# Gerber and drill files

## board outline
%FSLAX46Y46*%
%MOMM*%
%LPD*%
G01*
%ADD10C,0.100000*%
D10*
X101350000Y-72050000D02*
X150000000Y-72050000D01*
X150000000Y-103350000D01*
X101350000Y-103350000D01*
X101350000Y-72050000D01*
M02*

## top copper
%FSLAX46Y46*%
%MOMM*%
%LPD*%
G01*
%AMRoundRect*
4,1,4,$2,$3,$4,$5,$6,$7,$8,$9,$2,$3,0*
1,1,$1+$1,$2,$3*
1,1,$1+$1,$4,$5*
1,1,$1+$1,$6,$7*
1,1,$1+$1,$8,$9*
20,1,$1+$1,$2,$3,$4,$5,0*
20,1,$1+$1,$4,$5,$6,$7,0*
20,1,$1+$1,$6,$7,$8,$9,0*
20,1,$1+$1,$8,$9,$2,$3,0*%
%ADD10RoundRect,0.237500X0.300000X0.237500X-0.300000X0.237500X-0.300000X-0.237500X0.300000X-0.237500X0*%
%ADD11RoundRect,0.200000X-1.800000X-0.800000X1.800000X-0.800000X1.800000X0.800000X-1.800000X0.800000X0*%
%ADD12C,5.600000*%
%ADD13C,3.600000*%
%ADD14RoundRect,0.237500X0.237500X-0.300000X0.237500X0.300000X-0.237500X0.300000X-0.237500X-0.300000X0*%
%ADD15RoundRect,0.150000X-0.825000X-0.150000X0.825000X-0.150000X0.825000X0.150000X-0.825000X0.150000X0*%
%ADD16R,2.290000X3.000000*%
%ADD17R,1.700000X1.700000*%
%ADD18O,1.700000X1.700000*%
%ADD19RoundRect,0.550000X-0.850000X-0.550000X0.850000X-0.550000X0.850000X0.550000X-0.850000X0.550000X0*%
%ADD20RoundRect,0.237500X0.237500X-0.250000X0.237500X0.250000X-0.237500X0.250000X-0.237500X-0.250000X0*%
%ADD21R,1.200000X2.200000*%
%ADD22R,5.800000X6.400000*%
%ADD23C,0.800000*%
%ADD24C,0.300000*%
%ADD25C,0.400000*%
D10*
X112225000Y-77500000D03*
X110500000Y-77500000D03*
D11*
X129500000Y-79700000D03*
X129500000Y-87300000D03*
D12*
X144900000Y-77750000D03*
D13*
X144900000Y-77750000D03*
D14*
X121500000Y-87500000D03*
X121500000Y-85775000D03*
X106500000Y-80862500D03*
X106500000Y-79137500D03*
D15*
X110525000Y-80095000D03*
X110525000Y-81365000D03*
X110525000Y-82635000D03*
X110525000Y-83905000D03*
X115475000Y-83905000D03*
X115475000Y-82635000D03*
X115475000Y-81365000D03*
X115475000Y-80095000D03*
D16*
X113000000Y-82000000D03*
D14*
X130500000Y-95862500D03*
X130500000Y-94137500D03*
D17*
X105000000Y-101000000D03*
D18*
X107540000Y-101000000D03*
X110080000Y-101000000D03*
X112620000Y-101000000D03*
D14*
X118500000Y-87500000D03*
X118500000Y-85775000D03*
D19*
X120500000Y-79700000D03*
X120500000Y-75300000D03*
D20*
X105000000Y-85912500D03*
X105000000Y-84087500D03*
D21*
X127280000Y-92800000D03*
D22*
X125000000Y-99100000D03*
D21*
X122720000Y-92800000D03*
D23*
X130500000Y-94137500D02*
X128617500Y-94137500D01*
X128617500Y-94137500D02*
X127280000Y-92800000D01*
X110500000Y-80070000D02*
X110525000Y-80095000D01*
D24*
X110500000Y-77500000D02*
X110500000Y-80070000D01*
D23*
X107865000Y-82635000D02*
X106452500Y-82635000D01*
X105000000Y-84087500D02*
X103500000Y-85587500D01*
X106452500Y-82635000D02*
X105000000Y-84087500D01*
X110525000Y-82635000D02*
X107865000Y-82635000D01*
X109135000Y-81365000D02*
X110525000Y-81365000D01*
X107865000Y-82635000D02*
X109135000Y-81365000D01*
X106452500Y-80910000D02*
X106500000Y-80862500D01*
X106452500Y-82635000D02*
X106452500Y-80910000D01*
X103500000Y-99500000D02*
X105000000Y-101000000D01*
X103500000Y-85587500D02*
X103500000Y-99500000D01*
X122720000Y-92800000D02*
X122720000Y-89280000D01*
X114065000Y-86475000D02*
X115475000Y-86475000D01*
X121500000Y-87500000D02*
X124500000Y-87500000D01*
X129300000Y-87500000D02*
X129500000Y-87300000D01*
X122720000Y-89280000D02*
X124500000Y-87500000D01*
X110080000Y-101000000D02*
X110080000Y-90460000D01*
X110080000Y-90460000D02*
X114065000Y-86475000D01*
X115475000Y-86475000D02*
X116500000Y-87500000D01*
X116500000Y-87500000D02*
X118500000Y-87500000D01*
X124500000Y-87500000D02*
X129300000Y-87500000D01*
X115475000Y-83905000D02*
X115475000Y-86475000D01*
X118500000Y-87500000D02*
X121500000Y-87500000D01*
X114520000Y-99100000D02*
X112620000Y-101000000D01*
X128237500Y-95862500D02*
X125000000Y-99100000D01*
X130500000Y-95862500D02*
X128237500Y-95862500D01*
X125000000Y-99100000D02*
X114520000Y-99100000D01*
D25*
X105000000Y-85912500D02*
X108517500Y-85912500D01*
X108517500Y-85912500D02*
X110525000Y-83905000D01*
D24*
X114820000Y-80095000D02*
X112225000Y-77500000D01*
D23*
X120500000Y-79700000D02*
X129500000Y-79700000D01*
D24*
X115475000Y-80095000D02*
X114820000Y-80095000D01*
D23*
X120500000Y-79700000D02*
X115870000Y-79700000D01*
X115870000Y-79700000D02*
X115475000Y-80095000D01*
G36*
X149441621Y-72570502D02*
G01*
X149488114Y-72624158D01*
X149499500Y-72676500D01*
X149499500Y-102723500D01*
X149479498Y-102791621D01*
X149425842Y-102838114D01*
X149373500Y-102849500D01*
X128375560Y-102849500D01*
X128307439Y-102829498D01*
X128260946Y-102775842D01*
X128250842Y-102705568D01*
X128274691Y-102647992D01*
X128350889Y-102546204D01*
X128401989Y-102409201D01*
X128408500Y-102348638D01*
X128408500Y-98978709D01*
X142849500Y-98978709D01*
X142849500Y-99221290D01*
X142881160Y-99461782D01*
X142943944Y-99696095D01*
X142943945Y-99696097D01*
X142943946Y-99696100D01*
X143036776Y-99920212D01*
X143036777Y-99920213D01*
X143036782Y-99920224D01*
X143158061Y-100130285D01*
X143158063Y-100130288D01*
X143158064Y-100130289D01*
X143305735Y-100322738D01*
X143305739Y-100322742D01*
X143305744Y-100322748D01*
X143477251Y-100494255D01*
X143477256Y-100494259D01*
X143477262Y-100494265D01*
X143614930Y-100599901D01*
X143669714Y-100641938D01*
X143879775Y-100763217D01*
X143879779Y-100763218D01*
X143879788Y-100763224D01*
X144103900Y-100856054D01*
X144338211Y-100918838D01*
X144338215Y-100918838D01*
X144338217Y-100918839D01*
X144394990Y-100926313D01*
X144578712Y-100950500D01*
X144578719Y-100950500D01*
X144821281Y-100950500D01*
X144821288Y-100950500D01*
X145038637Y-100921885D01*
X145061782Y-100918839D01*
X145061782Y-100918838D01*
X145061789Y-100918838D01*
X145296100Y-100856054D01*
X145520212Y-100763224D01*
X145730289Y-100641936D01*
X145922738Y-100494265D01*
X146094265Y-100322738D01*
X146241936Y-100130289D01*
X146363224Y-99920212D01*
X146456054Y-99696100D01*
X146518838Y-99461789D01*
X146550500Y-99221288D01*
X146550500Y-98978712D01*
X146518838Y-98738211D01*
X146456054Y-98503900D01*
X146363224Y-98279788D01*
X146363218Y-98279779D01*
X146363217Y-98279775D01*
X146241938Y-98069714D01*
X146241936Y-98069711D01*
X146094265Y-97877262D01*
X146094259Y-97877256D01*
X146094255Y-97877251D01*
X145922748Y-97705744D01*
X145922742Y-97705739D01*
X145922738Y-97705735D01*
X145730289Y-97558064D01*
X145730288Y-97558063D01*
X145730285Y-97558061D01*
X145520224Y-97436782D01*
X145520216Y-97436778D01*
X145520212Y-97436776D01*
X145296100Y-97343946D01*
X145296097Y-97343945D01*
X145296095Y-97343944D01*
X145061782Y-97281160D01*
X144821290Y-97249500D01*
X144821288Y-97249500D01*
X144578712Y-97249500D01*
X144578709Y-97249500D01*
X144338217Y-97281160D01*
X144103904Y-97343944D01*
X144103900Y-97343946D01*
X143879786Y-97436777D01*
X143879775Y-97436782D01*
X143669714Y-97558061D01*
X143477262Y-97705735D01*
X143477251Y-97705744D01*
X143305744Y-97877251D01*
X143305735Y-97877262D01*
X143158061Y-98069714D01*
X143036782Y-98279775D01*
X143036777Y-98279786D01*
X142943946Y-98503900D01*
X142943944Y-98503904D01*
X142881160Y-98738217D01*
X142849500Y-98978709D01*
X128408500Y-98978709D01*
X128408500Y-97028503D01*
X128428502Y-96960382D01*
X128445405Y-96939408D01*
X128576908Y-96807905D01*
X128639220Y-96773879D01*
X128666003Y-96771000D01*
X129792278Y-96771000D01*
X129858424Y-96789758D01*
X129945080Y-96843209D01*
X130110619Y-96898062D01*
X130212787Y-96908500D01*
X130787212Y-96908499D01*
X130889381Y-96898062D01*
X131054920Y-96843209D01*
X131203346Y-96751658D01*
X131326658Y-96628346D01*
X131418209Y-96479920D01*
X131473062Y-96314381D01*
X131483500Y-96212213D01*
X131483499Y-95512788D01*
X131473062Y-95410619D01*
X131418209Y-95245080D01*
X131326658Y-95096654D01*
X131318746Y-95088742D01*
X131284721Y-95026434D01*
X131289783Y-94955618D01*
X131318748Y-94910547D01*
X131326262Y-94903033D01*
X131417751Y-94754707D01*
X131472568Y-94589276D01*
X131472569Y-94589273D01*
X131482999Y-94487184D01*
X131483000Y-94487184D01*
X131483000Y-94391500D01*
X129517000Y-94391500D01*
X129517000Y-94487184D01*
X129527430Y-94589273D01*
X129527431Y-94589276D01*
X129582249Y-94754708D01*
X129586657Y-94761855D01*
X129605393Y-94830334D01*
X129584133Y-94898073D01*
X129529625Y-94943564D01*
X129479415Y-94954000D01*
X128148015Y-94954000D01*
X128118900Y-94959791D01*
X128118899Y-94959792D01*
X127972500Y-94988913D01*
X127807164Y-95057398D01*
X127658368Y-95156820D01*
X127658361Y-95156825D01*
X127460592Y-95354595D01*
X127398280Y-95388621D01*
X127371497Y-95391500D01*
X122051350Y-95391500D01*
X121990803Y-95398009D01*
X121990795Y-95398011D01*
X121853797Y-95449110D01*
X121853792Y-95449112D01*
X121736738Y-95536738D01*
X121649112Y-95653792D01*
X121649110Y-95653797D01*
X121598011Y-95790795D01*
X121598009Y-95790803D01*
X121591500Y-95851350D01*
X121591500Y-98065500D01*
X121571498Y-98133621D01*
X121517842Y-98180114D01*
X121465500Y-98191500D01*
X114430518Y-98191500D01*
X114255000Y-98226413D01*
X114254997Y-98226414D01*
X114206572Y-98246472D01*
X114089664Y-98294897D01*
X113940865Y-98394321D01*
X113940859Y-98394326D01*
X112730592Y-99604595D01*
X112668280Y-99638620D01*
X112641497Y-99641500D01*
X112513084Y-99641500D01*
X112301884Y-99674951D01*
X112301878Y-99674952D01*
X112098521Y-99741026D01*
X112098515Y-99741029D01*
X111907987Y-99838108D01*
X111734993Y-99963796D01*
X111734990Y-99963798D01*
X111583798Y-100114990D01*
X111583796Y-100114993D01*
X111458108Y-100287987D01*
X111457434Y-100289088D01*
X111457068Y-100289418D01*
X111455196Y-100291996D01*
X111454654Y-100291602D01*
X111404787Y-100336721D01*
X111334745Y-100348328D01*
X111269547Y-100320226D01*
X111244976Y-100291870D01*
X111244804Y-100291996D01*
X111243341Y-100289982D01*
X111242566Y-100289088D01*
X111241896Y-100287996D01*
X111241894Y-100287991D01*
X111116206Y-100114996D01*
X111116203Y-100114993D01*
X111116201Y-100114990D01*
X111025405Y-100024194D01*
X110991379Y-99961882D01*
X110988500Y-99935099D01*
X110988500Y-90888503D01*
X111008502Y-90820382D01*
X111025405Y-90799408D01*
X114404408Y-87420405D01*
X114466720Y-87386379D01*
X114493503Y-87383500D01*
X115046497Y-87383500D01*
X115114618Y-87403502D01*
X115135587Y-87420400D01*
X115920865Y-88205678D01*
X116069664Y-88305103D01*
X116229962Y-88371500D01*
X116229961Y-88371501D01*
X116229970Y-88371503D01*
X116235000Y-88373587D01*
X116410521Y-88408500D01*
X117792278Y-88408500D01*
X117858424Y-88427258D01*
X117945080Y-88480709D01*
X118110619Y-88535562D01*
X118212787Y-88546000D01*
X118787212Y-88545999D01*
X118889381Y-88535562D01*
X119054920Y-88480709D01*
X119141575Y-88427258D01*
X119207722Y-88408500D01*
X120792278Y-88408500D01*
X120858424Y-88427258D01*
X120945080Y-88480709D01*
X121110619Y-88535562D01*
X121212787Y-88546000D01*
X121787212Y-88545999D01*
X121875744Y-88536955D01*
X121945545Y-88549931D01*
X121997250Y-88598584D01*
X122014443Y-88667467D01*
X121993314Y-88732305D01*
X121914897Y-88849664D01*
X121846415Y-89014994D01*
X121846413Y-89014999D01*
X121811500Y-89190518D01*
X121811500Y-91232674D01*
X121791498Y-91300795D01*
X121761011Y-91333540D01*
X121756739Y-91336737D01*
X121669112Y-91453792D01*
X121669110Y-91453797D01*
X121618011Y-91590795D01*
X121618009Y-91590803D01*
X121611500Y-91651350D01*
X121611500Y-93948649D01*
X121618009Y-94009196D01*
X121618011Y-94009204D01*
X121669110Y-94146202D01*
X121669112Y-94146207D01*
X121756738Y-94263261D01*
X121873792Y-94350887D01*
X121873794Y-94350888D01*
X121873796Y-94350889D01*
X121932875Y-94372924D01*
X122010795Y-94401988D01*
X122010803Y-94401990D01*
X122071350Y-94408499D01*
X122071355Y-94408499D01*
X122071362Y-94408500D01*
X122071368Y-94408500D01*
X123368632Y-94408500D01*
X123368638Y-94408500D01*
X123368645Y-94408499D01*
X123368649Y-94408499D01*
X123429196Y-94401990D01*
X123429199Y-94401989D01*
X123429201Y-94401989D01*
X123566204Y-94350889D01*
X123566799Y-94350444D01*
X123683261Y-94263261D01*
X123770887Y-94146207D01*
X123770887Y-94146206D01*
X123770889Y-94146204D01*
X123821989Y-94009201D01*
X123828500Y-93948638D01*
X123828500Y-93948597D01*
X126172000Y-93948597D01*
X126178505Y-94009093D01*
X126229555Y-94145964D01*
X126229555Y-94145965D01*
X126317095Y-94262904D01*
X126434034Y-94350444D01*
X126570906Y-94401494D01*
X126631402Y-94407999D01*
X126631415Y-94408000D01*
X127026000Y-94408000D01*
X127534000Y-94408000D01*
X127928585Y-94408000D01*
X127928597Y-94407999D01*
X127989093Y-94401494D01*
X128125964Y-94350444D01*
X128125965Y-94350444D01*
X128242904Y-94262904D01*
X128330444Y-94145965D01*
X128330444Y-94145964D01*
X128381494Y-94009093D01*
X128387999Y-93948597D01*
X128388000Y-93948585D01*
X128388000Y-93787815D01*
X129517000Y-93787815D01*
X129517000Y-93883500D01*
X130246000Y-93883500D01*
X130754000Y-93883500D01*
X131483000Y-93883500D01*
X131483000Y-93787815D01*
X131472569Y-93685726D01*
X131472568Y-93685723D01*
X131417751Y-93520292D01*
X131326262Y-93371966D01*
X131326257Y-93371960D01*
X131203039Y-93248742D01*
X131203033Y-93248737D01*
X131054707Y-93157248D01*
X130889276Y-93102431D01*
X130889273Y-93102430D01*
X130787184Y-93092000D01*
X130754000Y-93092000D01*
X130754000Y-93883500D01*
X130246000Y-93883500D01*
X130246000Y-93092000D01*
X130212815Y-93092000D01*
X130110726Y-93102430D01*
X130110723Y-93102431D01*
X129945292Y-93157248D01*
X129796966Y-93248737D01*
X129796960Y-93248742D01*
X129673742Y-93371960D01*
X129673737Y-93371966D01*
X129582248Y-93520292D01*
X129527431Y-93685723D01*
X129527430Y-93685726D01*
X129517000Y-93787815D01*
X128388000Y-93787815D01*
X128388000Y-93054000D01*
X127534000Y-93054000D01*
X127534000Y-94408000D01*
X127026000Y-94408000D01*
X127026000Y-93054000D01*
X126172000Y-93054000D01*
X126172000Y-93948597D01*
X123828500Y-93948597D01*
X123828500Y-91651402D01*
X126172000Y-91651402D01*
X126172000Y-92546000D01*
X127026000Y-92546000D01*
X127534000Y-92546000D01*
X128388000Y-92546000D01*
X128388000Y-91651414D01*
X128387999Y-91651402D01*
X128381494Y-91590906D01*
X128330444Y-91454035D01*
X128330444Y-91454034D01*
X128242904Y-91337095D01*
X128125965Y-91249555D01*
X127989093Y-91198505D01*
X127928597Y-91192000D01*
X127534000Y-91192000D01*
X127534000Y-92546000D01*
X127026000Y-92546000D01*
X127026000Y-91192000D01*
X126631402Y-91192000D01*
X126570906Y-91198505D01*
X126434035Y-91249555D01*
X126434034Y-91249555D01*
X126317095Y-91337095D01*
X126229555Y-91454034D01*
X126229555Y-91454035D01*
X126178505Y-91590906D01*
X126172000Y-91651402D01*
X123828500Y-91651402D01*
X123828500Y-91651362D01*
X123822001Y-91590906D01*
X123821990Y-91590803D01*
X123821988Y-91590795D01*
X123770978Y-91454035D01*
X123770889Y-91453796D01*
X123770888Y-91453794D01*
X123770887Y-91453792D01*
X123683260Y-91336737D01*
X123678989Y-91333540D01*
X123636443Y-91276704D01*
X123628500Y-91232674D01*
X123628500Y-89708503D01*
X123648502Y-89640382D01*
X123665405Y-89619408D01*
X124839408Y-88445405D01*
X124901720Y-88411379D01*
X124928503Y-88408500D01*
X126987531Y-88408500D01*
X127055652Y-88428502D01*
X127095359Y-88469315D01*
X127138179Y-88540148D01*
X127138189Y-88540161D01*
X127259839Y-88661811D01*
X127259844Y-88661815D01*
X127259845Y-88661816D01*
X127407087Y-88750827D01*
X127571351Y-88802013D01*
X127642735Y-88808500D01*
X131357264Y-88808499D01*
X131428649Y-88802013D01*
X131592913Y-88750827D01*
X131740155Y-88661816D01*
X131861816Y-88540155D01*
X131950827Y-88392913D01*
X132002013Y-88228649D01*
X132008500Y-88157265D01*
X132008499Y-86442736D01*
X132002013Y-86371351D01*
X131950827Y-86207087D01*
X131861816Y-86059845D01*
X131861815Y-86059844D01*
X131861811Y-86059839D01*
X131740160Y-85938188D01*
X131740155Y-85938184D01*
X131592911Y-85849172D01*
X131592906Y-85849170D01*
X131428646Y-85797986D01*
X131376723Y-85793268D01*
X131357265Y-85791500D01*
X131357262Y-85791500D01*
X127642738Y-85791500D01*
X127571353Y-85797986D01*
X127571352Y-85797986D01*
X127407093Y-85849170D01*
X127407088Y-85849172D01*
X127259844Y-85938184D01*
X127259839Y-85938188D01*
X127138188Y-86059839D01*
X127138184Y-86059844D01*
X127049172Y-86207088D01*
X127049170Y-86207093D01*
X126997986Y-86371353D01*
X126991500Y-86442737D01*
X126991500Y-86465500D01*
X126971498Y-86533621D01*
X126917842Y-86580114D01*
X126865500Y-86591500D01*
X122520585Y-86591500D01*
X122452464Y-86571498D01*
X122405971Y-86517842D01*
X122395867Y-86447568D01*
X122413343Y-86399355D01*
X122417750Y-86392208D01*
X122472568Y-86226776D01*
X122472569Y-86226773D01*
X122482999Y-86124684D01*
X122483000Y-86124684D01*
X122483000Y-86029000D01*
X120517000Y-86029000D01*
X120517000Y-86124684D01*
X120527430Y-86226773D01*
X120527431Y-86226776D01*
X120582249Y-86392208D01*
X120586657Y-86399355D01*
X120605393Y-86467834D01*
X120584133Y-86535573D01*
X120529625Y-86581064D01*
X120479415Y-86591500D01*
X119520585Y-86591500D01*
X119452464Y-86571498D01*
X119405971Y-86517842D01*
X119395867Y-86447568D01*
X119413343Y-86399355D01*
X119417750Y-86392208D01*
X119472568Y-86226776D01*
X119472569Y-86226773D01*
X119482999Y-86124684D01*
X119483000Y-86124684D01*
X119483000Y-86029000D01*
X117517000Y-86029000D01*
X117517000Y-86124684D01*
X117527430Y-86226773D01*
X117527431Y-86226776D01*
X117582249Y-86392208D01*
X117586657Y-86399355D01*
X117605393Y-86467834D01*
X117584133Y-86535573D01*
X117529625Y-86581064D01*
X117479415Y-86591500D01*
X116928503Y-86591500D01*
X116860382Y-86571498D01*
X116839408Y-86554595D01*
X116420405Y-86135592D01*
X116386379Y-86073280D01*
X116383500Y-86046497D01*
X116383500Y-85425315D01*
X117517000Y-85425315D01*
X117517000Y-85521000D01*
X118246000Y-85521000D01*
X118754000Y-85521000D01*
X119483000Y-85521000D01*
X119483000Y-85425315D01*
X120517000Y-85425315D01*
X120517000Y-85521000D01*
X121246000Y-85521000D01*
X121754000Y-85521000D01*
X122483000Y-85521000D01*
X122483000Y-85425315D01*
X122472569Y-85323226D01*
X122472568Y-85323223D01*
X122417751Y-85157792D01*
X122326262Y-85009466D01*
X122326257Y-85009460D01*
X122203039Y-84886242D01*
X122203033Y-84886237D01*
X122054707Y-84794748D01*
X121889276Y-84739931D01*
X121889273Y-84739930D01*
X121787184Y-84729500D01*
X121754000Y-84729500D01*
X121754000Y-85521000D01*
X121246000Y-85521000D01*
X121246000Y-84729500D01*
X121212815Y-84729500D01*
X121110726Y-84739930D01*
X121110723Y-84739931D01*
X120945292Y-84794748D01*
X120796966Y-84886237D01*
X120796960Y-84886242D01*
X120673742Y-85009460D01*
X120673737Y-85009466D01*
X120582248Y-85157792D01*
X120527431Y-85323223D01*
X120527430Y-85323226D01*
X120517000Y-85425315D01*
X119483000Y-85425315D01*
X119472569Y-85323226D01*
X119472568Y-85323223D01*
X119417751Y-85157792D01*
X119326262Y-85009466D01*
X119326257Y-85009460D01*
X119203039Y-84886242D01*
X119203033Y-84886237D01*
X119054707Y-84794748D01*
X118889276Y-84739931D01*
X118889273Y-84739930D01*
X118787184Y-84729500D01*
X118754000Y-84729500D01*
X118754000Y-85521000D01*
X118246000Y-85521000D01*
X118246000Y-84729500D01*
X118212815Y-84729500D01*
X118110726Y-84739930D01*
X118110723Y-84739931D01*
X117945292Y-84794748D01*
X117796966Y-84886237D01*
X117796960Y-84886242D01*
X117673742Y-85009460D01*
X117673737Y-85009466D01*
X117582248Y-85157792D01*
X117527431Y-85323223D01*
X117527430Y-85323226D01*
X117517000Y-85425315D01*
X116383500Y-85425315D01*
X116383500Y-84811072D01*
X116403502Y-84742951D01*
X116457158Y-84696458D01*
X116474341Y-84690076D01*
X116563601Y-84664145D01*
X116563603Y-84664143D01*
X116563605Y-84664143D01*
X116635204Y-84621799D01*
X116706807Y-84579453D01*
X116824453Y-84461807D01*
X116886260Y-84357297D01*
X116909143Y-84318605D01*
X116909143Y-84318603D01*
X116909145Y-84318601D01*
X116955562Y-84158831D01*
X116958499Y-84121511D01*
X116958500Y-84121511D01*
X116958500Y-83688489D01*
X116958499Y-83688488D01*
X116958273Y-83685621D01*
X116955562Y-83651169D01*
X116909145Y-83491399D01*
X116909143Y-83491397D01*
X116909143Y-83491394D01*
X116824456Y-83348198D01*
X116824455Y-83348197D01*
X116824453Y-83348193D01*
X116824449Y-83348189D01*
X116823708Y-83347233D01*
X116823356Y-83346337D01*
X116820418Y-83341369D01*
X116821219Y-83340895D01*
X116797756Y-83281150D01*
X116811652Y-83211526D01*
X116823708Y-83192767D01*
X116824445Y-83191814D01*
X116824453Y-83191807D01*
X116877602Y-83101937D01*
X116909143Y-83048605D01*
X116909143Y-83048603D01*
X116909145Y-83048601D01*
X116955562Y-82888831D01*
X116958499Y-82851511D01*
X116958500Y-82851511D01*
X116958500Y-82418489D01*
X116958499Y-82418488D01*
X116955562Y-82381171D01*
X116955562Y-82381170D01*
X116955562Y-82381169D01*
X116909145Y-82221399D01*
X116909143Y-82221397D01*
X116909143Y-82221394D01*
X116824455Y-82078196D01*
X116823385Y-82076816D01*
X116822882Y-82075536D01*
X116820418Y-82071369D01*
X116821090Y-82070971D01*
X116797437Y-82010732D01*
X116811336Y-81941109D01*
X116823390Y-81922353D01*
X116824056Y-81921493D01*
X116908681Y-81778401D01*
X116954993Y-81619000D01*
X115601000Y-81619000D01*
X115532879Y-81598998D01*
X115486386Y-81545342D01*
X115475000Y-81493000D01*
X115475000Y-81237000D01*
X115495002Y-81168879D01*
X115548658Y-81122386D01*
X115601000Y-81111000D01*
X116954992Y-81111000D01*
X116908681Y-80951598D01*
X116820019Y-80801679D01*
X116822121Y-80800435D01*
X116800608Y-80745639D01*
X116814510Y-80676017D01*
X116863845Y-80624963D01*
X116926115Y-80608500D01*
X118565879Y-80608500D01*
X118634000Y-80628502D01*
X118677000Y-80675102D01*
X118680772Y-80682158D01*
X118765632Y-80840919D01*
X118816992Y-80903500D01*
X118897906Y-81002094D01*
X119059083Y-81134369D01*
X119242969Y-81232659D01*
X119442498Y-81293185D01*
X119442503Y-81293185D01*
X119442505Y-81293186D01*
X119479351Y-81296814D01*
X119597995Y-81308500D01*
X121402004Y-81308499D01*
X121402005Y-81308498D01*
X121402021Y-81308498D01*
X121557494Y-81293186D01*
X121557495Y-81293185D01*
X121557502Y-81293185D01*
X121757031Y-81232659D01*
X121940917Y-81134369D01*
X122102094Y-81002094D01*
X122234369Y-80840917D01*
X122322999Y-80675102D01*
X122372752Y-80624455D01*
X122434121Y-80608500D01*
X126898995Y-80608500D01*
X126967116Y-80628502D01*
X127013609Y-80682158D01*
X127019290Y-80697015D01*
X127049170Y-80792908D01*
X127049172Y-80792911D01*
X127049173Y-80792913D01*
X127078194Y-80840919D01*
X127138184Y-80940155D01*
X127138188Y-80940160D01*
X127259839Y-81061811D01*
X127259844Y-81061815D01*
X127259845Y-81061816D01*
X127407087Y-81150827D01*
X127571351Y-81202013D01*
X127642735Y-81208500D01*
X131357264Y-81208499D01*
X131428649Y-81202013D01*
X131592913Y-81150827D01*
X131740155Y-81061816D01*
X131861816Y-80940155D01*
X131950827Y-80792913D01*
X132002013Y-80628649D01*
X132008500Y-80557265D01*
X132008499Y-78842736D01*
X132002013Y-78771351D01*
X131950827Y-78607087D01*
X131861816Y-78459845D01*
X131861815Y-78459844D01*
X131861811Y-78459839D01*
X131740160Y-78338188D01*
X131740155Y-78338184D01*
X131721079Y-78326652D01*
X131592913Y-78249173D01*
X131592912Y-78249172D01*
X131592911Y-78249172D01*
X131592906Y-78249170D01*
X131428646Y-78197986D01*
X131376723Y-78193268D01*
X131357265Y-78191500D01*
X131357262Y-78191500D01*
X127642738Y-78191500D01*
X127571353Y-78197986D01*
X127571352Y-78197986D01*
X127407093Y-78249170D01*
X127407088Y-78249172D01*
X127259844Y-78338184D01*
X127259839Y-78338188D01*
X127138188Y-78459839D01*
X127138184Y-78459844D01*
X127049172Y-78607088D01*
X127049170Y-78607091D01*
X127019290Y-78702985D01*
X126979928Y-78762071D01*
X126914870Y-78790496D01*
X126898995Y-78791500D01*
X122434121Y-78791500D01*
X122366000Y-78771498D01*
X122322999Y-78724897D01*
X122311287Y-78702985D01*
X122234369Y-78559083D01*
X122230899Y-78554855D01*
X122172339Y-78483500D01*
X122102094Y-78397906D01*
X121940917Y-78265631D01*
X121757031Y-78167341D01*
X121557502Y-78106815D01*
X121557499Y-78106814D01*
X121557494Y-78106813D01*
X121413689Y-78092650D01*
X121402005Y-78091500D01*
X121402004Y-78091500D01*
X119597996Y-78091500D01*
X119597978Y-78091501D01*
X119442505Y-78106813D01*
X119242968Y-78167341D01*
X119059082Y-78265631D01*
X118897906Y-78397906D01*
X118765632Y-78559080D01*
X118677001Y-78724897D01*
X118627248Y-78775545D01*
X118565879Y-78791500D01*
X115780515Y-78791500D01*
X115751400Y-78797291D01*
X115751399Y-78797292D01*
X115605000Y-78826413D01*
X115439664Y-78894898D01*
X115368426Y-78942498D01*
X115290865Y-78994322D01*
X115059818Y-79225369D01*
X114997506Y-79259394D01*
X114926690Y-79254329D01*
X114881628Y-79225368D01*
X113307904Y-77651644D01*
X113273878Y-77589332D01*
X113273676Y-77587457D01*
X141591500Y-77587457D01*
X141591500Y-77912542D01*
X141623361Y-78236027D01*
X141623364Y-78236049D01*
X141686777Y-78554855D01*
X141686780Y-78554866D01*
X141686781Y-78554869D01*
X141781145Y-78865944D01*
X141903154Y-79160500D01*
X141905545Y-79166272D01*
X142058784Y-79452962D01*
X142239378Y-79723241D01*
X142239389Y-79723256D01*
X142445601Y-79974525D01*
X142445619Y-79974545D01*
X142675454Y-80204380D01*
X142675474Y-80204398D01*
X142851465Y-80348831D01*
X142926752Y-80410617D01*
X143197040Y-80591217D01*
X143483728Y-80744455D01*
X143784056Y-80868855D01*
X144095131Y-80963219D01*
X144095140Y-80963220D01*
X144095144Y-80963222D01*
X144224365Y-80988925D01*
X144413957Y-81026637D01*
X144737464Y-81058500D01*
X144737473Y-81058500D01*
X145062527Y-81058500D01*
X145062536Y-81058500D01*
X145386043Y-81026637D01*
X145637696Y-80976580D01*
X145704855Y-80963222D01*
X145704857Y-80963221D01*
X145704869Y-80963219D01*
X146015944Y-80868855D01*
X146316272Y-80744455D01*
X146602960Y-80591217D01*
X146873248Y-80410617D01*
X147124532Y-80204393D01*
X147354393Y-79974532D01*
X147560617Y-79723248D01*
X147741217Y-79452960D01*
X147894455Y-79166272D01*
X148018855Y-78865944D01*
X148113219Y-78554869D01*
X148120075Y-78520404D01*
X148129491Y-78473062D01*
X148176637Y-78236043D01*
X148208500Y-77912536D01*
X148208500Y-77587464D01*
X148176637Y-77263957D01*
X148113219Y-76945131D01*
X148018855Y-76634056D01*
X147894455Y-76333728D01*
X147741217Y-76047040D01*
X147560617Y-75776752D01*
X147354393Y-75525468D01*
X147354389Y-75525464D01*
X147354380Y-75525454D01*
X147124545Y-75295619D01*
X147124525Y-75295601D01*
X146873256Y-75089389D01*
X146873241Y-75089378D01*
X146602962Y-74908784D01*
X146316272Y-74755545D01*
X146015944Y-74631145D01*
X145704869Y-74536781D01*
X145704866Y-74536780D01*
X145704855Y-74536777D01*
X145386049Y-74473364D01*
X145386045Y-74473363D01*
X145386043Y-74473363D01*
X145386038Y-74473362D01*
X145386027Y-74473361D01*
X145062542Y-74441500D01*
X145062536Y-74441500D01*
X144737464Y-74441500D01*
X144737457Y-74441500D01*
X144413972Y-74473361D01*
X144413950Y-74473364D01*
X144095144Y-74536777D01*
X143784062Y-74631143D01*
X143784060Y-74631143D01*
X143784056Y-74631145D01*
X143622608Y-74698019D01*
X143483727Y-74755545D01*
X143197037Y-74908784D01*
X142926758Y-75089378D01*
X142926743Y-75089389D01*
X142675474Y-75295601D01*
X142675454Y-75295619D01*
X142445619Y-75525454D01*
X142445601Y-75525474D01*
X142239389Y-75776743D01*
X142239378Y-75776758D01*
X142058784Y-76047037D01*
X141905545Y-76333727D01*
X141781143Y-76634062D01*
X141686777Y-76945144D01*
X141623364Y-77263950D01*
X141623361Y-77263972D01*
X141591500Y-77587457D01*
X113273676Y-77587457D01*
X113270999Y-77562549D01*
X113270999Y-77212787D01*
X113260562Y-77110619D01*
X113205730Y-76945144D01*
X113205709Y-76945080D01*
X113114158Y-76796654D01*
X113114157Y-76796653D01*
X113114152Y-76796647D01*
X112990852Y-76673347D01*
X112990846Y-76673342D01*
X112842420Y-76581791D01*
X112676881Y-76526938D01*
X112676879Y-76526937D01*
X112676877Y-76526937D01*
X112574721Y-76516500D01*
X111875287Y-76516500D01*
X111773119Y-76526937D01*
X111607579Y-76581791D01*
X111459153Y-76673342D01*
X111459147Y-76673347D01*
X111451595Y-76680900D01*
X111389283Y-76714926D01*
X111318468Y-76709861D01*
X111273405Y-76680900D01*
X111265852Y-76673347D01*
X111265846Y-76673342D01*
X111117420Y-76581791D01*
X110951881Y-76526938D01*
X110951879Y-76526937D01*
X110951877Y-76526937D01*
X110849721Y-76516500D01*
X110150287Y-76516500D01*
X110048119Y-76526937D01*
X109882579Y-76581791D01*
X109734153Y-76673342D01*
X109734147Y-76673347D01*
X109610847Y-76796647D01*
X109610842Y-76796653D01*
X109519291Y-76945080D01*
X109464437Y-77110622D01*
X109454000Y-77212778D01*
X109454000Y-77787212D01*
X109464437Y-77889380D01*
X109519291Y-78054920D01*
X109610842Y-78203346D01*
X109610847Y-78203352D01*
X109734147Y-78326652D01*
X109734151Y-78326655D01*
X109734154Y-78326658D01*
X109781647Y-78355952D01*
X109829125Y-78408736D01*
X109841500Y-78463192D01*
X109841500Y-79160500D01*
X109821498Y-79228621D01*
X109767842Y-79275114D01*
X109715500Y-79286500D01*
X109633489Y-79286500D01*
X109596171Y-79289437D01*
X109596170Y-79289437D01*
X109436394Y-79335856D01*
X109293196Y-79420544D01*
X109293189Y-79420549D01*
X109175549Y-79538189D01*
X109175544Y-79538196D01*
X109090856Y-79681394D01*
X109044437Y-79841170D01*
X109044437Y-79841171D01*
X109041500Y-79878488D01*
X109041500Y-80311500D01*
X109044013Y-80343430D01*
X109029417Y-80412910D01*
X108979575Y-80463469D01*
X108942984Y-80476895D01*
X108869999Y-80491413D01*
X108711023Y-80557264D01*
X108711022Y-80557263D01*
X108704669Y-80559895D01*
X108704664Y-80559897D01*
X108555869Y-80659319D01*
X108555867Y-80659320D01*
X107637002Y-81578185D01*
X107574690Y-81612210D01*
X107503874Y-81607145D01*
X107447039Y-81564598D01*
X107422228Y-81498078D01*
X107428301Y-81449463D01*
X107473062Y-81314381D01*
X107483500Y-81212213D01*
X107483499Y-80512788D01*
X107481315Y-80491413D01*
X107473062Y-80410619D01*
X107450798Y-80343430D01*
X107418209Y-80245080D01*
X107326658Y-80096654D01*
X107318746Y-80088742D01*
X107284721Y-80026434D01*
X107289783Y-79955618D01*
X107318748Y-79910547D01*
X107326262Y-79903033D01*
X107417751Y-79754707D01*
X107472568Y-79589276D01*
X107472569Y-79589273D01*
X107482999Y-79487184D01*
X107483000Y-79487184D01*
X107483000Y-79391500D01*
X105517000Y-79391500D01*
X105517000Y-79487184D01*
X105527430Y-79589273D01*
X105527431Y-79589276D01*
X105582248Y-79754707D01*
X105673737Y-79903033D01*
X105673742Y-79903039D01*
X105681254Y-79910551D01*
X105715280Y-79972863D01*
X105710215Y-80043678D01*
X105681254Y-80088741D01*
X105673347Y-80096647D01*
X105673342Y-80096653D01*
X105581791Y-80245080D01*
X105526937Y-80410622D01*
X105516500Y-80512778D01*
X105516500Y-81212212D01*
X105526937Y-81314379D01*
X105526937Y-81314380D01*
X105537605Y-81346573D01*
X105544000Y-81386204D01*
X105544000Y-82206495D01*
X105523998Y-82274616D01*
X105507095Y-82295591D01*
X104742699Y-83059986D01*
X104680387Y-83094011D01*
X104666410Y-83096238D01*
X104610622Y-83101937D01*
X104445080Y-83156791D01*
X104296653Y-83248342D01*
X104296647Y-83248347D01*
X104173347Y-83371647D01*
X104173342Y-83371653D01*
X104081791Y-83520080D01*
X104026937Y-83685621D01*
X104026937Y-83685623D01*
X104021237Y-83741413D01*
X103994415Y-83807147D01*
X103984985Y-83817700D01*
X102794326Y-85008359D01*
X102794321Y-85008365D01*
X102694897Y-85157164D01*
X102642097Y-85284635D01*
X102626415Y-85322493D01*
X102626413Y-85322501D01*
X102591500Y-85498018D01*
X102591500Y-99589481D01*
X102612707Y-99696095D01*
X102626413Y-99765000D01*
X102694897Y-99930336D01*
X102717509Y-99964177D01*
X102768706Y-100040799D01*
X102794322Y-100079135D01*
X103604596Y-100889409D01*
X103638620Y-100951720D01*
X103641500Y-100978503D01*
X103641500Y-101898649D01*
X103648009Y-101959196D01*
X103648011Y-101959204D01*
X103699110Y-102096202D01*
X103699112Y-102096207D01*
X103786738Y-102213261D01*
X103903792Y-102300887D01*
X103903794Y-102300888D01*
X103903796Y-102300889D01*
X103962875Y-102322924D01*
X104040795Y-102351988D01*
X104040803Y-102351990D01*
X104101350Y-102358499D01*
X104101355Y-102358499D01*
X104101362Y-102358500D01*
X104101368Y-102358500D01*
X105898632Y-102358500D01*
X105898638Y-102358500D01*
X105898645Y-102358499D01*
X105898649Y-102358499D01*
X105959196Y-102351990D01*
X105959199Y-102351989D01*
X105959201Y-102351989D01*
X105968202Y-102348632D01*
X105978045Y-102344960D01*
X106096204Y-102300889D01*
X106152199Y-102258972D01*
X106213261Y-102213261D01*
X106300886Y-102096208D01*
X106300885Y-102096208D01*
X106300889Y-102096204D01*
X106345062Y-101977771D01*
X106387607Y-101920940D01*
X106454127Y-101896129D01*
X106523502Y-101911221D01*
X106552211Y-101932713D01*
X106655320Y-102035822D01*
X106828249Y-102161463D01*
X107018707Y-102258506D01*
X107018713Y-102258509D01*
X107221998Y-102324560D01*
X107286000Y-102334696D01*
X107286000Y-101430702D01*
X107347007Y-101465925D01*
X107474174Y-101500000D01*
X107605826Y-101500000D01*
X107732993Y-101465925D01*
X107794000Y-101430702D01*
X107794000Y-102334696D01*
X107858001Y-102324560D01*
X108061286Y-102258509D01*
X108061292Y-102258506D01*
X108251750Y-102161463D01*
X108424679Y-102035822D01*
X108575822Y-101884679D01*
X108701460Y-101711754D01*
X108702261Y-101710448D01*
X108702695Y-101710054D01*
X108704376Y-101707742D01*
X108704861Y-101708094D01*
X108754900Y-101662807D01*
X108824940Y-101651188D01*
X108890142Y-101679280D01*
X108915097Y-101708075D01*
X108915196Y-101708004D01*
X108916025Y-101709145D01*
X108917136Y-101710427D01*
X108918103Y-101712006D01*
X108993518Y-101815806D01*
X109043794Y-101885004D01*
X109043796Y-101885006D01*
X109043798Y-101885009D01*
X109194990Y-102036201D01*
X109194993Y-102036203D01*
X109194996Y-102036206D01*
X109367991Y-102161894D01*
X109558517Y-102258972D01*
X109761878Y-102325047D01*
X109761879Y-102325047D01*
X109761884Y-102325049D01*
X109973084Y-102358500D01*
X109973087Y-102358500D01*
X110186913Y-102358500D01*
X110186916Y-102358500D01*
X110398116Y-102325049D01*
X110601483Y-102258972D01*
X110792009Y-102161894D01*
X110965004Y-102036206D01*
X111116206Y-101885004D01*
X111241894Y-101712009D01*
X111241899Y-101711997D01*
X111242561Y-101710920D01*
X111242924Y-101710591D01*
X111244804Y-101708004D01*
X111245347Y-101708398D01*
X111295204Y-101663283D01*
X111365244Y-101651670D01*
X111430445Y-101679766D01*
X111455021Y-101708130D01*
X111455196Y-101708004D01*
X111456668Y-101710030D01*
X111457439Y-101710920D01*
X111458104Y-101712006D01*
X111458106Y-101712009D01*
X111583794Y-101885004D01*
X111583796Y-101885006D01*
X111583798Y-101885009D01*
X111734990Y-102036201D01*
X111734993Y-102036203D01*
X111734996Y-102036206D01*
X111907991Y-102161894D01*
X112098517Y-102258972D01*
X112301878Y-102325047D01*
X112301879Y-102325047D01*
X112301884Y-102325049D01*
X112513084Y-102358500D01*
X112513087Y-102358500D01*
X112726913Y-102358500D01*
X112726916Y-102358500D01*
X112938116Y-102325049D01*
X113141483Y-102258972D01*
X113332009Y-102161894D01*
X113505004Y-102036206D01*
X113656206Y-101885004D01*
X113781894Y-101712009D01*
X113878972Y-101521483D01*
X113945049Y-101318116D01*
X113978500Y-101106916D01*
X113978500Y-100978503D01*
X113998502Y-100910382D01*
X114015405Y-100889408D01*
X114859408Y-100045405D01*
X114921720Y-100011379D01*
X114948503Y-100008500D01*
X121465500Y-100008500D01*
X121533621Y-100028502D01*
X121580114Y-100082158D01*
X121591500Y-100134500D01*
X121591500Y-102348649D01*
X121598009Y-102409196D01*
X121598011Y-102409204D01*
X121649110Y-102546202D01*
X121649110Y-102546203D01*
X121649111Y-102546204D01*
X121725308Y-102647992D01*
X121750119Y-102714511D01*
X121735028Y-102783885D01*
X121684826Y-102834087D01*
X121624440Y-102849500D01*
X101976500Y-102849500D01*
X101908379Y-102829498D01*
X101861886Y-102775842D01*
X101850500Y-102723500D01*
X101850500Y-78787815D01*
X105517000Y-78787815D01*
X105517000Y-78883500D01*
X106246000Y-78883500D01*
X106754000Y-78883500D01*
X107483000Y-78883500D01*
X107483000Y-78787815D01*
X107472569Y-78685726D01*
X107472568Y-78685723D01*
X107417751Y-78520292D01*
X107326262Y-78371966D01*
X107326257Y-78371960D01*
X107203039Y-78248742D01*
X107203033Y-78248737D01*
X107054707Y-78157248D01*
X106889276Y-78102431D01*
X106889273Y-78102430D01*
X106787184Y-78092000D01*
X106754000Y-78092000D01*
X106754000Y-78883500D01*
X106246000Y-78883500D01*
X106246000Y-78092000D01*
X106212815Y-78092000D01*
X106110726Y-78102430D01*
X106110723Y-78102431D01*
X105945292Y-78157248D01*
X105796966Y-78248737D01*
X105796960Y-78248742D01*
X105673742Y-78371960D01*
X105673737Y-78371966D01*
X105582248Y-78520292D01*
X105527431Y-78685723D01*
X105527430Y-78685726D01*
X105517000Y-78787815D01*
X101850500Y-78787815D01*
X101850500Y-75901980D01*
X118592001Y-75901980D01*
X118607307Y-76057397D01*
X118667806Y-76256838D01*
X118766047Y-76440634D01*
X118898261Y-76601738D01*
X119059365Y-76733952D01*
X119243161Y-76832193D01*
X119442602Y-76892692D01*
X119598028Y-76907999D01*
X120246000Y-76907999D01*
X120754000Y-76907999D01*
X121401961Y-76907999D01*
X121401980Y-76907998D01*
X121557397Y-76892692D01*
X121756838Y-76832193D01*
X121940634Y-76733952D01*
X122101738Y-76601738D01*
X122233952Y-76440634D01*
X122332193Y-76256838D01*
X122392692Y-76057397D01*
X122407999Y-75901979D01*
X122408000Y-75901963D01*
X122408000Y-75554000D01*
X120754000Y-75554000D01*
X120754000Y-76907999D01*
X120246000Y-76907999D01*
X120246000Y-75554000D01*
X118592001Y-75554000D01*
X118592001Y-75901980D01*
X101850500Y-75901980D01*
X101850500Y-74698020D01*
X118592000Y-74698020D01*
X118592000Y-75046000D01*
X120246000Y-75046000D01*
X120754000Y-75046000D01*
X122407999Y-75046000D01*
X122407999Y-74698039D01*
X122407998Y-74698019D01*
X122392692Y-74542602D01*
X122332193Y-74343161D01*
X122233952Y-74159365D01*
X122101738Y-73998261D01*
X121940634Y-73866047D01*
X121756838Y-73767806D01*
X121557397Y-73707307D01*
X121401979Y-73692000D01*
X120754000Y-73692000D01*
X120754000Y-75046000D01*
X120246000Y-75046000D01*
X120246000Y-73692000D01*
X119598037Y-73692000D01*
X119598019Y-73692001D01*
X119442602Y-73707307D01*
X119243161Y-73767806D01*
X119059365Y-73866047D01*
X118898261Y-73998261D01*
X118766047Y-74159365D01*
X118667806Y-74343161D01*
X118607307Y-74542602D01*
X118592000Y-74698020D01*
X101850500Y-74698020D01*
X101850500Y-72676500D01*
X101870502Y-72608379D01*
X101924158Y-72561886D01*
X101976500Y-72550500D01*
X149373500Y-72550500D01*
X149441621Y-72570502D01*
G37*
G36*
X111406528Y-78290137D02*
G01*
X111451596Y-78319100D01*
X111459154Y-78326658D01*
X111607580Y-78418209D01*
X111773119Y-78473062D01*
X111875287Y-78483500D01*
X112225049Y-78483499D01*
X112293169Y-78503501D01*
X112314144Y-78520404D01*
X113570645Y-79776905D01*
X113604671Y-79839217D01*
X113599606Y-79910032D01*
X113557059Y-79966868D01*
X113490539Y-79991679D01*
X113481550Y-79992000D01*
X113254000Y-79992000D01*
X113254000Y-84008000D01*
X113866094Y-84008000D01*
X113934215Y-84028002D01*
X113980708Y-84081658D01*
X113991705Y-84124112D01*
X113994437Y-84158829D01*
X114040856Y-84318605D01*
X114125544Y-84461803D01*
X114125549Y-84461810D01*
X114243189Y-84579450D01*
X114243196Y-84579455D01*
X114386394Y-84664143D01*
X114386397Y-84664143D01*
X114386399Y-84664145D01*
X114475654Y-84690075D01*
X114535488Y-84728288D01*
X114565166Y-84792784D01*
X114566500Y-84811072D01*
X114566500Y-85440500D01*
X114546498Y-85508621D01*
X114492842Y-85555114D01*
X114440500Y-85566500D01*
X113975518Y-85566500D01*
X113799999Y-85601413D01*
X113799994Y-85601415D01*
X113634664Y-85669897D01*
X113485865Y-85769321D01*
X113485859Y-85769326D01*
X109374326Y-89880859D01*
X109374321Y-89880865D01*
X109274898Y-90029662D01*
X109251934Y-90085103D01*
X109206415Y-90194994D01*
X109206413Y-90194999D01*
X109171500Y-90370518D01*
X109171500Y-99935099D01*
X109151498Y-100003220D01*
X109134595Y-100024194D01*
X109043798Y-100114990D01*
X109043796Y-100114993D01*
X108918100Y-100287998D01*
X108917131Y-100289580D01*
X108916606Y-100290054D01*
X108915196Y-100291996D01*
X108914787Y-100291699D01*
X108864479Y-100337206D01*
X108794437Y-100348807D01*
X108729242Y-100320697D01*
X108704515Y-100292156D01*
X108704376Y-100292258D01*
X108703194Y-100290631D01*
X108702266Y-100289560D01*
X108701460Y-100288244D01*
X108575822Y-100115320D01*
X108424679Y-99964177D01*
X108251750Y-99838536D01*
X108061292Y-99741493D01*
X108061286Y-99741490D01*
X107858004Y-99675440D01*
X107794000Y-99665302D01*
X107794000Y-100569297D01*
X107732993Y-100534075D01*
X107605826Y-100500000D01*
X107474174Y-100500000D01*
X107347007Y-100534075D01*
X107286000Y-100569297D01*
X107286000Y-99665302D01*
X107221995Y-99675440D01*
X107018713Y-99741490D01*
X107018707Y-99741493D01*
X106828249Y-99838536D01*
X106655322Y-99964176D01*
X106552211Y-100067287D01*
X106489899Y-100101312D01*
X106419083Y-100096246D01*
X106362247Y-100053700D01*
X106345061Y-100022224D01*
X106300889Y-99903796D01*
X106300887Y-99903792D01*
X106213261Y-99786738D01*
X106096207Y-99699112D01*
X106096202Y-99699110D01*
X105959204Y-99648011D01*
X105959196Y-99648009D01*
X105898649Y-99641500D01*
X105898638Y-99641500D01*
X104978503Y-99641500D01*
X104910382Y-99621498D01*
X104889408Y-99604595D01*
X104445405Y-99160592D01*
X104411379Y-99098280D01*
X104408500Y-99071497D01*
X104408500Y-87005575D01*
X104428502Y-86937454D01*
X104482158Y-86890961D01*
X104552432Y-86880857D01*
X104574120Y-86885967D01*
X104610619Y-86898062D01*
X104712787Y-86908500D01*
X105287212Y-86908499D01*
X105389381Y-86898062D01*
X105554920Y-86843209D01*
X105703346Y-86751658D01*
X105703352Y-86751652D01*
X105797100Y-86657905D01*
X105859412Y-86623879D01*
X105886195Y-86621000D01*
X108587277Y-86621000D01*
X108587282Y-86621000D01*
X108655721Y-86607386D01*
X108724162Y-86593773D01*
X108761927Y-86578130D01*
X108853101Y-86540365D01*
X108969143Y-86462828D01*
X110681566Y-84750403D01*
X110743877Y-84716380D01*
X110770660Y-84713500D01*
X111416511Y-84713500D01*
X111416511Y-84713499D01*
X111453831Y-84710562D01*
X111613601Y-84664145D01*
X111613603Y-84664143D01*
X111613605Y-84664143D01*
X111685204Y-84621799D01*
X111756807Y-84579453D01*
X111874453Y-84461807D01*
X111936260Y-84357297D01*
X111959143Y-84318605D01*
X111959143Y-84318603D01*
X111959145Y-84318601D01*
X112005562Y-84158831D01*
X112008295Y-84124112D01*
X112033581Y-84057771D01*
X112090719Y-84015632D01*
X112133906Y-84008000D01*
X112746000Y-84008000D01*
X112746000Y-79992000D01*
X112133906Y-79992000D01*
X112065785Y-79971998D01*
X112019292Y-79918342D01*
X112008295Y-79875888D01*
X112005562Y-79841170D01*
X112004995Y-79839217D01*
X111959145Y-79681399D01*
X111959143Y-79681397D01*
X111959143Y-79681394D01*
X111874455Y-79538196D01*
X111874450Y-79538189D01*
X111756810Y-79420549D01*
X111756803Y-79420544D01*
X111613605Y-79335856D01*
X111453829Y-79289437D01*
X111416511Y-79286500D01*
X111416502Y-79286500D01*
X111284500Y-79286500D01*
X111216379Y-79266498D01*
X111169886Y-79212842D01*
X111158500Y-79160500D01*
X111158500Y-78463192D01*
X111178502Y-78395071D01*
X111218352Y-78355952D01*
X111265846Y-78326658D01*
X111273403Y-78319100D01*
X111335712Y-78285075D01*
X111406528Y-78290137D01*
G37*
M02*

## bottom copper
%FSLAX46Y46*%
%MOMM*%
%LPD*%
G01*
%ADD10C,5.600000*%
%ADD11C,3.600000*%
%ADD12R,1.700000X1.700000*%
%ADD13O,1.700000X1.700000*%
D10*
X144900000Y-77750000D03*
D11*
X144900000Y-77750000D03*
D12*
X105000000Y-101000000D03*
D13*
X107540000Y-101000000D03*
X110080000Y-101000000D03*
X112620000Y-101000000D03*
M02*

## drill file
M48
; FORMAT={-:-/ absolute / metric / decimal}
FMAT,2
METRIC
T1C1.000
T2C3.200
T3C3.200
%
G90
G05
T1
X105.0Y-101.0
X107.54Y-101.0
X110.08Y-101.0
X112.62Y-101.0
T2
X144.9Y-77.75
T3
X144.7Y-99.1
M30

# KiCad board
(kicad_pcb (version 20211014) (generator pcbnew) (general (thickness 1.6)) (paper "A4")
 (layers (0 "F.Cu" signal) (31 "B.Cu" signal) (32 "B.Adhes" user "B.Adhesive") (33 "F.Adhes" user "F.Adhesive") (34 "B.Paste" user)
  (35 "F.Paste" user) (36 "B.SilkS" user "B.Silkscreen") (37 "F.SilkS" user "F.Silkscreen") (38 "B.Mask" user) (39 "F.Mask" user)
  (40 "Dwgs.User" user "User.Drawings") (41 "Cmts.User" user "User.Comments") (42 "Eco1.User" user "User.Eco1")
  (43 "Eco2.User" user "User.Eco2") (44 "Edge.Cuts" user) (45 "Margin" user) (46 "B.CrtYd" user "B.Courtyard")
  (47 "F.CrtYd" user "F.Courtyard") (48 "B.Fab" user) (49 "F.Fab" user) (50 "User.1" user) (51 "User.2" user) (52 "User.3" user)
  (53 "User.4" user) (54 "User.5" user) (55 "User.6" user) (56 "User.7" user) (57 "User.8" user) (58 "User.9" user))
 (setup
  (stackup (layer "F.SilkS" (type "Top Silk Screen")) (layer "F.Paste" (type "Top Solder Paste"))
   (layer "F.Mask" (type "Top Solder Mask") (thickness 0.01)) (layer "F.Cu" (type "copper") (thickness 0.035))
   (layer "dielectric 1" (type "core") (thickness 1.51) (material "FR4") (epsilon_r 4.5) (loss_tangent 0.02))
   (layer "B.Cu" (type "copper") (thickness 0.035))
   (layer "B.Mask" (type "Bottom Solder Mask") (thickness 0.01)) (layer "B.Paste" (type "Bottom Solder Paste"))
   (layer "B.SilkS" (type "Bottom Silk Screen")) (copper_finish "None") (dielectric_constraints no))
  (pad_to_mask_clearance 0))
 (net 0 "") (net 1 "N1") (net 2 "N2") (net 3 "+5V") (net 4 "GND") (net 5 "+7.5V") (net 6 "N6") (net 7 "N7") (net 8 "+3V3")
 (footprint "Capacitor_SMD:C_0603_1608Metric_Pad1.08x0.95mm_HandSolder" (layer "F.Cu") (at 111.3625 77.5 180)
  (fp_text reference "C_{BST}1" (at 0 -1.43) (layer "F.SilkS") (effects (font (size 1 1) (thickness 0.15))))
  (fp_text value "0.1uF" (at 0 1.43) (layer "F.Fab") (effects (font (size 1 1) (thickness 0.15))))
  (pad "1" smd roundrect (at -0.8625 0 180) (size 1.075 0.95) (layers "F.Cu" "F.Paste" "F.Mask") (roundrect_rratio 0.25) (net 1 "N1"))
  (pad "2" smd roundrect (at 0.8625 0 180) (size 1.075 0.95) (layers "F.Cu" "F.Paste" "F.Mask") (roundrect_rratio 0.25) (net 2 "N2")))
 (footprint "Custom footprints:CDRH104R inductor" (layer "F.Cu") (at 129.5 83.5)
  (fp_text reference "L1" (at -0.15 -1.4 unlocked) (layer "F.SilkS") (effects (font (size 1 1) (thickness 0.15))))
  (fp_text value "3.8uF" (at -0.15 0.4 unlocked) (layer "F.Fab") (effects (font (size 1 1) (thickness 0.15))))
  (pad "1" smd roundrect (at 0 -3.8) (size 4 2) (layers "F.Cu" "F.Paste" "F.Mask") (roundrect_rratio 0.1) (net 1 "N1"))
  (pad "2" smd roundrect (at 0 3.8) (size 4 2) (layers "F.Cu" "F.Paste" "F.Mask") (roundrect_rratio 0.1) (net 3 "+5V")))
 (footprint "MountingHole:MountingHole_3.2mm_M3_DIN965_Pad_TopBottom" (layer "F.Cu") (at 144.9 77.75)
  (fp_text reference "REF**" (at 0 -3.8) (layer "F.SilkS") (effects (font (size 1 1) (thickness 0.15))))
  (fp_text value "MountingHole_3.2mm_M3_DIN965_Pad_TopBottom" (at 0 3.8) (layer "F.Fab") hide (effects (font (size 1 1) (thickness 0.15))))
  (pad "1" connect circle (at 0 0) (size 5.6 5.6) (layers "B.Cu" "B.Mask"))
  (pad "1" connect circle (at 0 0) (size 5.6 5.6) (layers "F.Cu" "F.Mask"))
  (pad "1" thru_hole circle (at 0 0) (size 3.6 3.6) (drill 3.2) (layers *.Cu *.Mask)))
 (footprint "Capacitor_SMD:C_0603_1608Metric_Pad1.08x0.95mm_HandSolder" (layer "F.Cu") (at 121.5 86.6375 90)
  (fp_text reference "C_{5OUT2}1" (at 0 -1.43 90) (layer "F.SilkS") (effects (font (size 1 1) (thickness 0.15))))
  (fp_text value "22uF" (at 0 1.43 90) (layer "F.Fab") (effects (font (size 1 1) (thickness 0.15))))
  (pad "1" smd roundrect (at -0.8625 0 90) (size 1.075 0.95) (layers "F.Cu" "F.Paste" "F.Mask") (roundrect_rratio 0.25) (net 3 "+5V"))
  (pad "2" smd roundrect (at 0.8625 0 90) (size 1.075 0.95) (layers "F.Cu" "F.Paste" "F.Mask") (roundrect_rratio 0.25) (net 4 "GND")))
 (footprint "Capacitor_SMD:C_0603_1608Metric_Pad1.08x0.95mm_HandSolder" (layer "F.Cu") (at 106.5 80 90)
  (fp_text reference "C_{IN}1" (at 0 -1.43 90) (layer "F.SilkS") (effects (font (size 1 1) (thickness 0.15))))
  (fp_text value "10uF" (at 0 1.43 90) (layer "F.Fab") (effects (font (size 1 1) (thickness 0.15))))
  (pad "1" smd roundrect (at -0.8625 0 90) (size 1.075 0.95) (layers "F.Cu" "F.Paste" "F.Mask") (roundrect_rratio 0.25) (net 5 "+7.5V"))
  (pad "2" smd roundrect (at 0.8625 0 90) (size 1.075 0.95) (layers "F.Cu" "F.Paste" "F.Mask") (roundrect_rratio 0.25) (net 4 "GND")))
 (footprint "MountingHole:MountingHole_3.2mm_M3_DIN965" (layer "F.Cu") (at 144.7 99.1)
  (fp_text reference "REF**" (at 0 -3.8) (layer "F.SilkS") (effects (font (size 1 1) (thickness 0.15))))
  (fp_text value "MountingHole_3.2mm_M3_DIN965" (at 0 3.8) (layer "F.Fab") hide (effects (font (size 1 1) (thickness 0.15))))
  (pad "" np_thru_hole circle (at 0 0) (size 3.2 3.2) (drill 3.2) (layers *.Cu *.Mask)))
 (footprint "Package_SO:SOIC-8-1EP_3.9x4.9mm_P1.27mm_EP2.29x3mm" (layer "F.Cu") (at 113 82)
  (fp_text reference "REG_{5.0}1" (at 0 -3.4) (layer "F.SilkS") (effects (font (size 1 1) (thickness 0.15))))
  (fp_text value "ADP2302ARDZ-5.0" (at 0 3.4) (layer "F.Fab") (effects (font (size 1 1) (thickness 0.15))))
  (pad "" smd roundrect (at 0.57 -0.75) (size 0.92 1.21) (layers "F.Paste") (roundrect_rratio 0.25))
  (pad "" smd roundrect (at 0.57 0.75) (size 0.92 1.21) (layers "F.Paste") (roundrect_rratio 0.25))
  (pad "" smd roundrect (at -0.57 -0.75) (size 0.92 1.21) (layers "F.Paste") (roundrect_rratio 0.25))
  (pad "" smd roundrect (at -0.57 0.75) (size 0.92 1.21) (layers "F.Paste") (roundrect_rratio 0.25))
  (pad "1" smd roundrect (at -2.475 -1.905) (size 1.95 0.6) (layers "F.Cu" "F.Paste" "F.Mask") (roundrect_rratio 0.25) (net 2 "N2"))
  (pad "2" smd roundrect (at -2.475 -0.635) (size 1.95 0.6) (layers "F.Cu" "F.Paste" "F.Mask") (roundrect_rratio 0.25) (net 5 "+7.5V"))
  (pad "3" smd roundrect (at -2.475 0.635) (size 1.95 0.6) (layers "F.Cu" "F.Paste" "F.Mask") (roundrect_rratio 0.25) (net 5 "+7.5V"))
  (pad "4" smd roundrect (at -2.475 1.905) (size 1.95 0.6) (layers "F.Cu" "F.Paste" "F.Mask") (roundrect_rratio 0.25) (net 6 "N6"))
  (pad "5" smd roundrect (at 2.475 1.905) (size 1.95 0.6) (layers "F.Cu" "F.Paste" "F.Mask") (roundrect_rratio 0.25) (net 3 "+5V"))
  (pad "6" smd roundrect (at 2.475 0.635) (size 1.95 0.6) (layers "F.Cu" "F.Paste" "F.Mask") (roundrect_rratio 0.25) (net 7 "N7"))
  (pad "7" smd roundrect (at 2.475 -0.635) (size 1.95 0.6) (layers "F.Cu" "F.Paste" "F.Mask") (roundrect_rratio 0.25) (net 4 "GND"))
  (pad "8" smd roundrect (at 2.475 -1.905) (size 1.95 0.6) (layers "F.Cu" "F.Paste" "F.Mask") (roundrect_rratio 0.25) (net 1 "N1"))
  (pad "9" smd rect (at 0 0) (size 2.29 3) (layers "F.Cu" "F.Mask") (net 4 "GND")))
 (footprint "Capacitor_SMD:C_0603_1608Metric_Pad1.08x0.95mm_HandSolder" (layer "F.Cu") (at 130.5 95 90)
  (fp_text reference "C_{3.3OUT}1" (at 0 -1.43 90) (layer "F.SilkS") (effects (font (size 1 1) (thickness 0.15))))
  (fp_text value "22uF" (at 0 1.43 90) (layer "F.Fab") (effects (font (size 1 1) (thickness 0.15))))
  (pad "1" smd roundrect (at -0.8625 0 90) (size 1.075 0.95) (layers "F.Cu" "F.Paste" "F.Mask") (roundrect_rratio 0.25) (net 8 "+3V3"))
  (pad "2" smd roundrect (at 0.8625 0 90) (size 1.075 0.95) (layers "F.Cu" "F.Paste" "F.Mask") (roundrect_rratio 0.25) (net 4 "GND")))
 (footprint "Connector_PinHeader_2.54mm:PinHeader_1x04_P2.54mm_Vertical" (layer "F.Cu") (at 105 101 90)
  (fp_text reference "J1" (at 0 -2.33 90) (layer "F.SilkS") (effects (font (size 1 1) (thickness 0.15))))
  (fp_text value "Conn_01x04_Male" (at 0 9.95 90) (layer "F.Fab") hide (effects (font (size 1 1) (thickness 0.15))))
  (pad "1" thru_hole rect (at 0 0 90) (size 1.7 1.7) (drill 1) (layers *.Cu *.Mask) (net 5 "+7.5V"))
  (pad "2" thru_hole oval (at 0 2.54 90) (size 1.7 1.7) (drill 1) (layers *.Cu *.Mask) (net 4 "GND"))
  (pad "3" thru_hole oval (at 0 5.08 90) (size 1.7 1.7) (drill 1) (layers *.Cu *.Mask) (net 3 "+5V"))
  (pad "4" thru_hole oval (at 0 7.62 90) (size 1.7 1.7) (drill 1) (layers *.Cu *.Mask) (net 8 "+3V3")))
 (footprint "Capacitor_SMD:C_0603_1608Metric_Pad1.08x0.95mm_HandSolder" (layer "F.Cu") (at 118.5 86.6375 90)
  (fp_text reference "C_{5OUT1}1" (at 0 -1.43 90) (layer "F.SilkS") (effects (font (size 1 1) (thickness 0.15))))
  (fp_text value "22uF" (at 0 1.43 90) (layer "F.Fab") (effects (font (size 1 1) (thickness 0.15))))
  (pad "1" smd roundrect (at -0.8625 0 90) (size 1.075 0.95) (layers "F.Cu" "F.Paste" "F.Mask") (roundrect_rratio 0.25) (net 3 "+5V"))
  (pad "2" smd roundrect (at 0.8625 0 90) (size 1.075 0.95) (layers "F.Cu" "F.Paste" "F.Mask") (roundrect_rratio 0.25) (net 4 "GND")))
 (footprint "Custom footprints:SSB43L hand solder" (layer "F.Cu") (at 120.5 77.5 -90)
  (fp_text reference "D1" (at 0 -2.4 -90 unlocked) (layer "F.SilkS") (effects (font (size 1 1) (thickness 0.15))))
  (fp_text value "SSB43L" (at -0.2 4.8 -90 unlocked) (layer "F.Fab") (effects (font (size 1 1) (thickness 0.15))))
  (pad "1" smd roundrect (at 2.2 0) (size 2.8 2.2) (layers "F.Cu" "F.Paste" "F.Mask") (roundrect_rratio 0.25) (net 1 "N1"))
  (pad "2" smd roundrect (at -2.2 0) (size 2.8 2.2) (layers "F.Cu" "F.Paste" "F.Mask") (roundrect_rratio 0.25) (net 4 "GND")))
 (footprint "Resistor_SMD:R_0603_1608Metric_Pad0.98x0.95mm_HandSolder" (layer "F.Cu") (at 105 85 90)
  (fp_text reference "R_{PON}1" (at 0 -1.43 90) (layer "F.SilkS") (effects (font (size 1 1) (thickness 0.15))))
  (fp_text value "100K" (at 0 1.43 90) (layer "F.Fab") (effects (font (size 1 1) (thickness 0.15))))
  (pad "1" smd roundrect (at -0.9125 0 90) (size 0.975 0.95) (layers "F.Cu" "F.Paste" "F.Mask") (roundrect_rratio 0.25) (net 6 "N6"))
  (pad "2" smd roundrect (at 0.9125 0 90) (size 0.975 0.95) (layers "F.Cu" "F.Paste" "F.Mask") (roundrect_rratio 0.25) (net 5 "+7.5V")))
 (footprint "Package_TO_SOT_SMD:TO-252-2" (layer "F.Cu") (at 125 97 -90)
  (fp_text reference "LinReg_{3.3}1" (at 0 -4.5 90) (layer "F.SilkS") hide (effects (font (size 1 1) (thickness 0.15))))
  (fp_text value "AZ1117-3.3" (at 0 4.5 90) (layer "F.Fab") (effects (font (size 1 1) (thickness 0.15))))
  (pad "" smd rect (at 0.425 1.525 270) (size 3.05 2.75) (layers "F.Paste"))
  (pad "" smd rect (at 0.425 -1.525 270) (size 3.05 2.75) (layers "F.Paste"))
  (pad "" smd rect (at 3.775 1.525 270) (size 3.05 2.75) (layers "F.Paste"))
  (pad "" smd rect (at 3.775 -1.525 270) (size 3.05 2.75) (layers "F.Paste"))
  (pad "1" smd rect (at -4.2 -2.28 270) (size 2.2 1.2) (layers "F.Cu" "F.Paste" "F.Mask") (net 4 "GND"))
  (pad "2" smd rect (at 2.1 0 270) (size 6.4 5.8) (layers "F.Cu" "F.Mask") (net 8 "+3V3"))
  (pad "3" smd rect (at -4.2 2.28 270) (size 2.2 1.2) (layers "F.Cu" "F.Paste" "F.Mask") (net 3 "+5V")))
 (gr_rect (start 101.35 103.35) (end 150 72.05) (layer "Edge.Cuts") (width 0.1) (fill none))
 (segment (start 130.5 94.1375) (end 128.6175 94.1375) (width 0.8) (layer "F.Cu") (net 4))
 (segment (start 128.6175 94.1375) (end 127.28 92.8) (width 0.8) (layer "F.Cu") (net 4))
 (segment (start 110.5 80.07) (end 110.525 80.095) (width 0.8) (layer "F.Cu") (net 2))
 (segment (start 110.5 77.5) (end 110.5 80.07) (width 0.3) (layer "F.Cu") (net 2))
 (segment (start 107.865 82.635) (end 106.4525 82.635) (width 0.8) (layer "F.Cu") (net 5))
 (segment (start 105 84.0875) (end 103.5 85.5875) (width 0.8) (layer "F.Cu") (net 5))
 (segment (start 106.4525 82.635) (end 105 84.0875) (width 0.8) (layer "F.Cu") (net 5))
 (segment (start 110.525 82.635) (end 107.865 82.635) (width 0.8) (layer "F.Cu") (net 5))
 (segment (start 109.135 81.365) (end 110.525 81.365) (width 0.8) (layer "F.Cu") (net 5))
 (segment (start 107.865 82.635) (end 109.135 81.365) (width 0.8) (layer "F.Cu") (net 5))
 (segment (start 106.4525 80.91) (end 106.5 80.8625) (width 0.8) (layer "F.Cu") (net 5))
 (segment (start 106.4525 82.635) (end 106.4525 80.91) (width 0.8) (layer "F.Cu") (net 5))
 (segment (start 103.5 99.5) (end 105 101) (width 0.8) (layer "F.Cu") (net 5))
 (segment (start 103.5 85.5875) (end 103.5 99.5) (width 0.8) (layer "F.Cu") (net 5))
 (segment (start 122.72 92.8) (end 122.72 89.28) (width 0.8) (layer "F.Cu") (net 3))
 (segment (start 114.065 86.475) (end 115.475 86.475) (width 0.8) (layer "F.Cu") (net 3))
 (segment (start 121.5 87.5) (end 124.5 87.5) (width 0.8) (layer "F.Cu") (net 3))
 (segment (start 129.3 87.5) (end 129.5 87.3) (width 0.8) (layer "F.Cu") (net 3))
 (segment (start 122.72 89.28) (end 124.5 87.5) (width 0.8) (layer "F.Cu") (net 3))
 (segment (start 110.08 101) (end 110.08 90.46) (width 0.8) (layer "F.Cu") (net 3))
 (segment (start 110.08 90.46) (end 114.065 86.475) (width 0.8) (layer "F.Cu") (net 3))
 (segment (start 115.475 86.475) (end 116.5 87.5) (width 0.8) (layer "F.Cu") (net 3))
 (segment (start 116.5 87.5) (end 118.5 87.5) (width 0.8) (layer "F.Cu") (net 3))
 (segment (start 124.5 87.5) (end 129.3 87.5) (width 0.8) (layer "F.Cu") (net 3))
 (segment (start 115.475 83.905) (end 115.475 86.475) (width 0.8) (layer "F.Cu") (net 3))
 (segment (start 118.5 87.5) (end 121.5 87.5) (width 0.8) (layer "F.Cu") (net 3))
 (segment (start 114.52 99.1) (end 112.62 101) (width 0.8) (layer "F.Cu") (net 8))
 (segment (start 128.2375 95.8625) (end 125 99.1) (width 0.8) (layer "F.Cu") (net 8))
 (segment (start 130.5 95.8625) (end 128.2375 95.8625) (width 0.8) (layer "F.Cu") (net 8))
 (segment (start 125 99.1) (end 114.52 99.1) (width 0.8) (layer "F.Cu") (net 8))
 (segment (start 105 85.9125) (end 108.5175 85.9125) (width 0.4) (layer "F.Cu") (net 6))
 (segment (start 108.5175 85.9125) (end 110.525 83.905) (width 0.4) (layer "F.Cu") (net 6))
 (segment (start 114.82 80.095) (end 112.225 77.5) (width 0.3) (layer "F.Cu") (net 1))
 (segment (start 120.5 79.7) (end 129.5 79.7) (width 0.8) (layer "F.Cu") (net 1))
 (segment (start 115.475 80.095) (end 114.82 80.095) (width 0.3) (layer "F.Cu") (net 1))
 (segment (start 120.5 79.7) (end 115.87 79.7) (width 0.8) (layer "F.Cu") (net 1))
 (segment (start 115.87 79.7) (end 115.475 80.095) (width 0.8) (layer "F.Cu") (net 1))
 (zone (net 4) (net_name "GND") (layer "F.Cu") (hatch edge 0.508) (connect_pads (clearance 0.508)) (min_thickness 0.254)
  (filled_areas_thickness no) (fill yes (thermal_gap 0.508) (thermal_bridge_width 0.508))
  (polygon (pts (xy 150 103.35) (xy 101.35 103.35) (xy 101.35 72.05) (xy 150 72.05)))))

